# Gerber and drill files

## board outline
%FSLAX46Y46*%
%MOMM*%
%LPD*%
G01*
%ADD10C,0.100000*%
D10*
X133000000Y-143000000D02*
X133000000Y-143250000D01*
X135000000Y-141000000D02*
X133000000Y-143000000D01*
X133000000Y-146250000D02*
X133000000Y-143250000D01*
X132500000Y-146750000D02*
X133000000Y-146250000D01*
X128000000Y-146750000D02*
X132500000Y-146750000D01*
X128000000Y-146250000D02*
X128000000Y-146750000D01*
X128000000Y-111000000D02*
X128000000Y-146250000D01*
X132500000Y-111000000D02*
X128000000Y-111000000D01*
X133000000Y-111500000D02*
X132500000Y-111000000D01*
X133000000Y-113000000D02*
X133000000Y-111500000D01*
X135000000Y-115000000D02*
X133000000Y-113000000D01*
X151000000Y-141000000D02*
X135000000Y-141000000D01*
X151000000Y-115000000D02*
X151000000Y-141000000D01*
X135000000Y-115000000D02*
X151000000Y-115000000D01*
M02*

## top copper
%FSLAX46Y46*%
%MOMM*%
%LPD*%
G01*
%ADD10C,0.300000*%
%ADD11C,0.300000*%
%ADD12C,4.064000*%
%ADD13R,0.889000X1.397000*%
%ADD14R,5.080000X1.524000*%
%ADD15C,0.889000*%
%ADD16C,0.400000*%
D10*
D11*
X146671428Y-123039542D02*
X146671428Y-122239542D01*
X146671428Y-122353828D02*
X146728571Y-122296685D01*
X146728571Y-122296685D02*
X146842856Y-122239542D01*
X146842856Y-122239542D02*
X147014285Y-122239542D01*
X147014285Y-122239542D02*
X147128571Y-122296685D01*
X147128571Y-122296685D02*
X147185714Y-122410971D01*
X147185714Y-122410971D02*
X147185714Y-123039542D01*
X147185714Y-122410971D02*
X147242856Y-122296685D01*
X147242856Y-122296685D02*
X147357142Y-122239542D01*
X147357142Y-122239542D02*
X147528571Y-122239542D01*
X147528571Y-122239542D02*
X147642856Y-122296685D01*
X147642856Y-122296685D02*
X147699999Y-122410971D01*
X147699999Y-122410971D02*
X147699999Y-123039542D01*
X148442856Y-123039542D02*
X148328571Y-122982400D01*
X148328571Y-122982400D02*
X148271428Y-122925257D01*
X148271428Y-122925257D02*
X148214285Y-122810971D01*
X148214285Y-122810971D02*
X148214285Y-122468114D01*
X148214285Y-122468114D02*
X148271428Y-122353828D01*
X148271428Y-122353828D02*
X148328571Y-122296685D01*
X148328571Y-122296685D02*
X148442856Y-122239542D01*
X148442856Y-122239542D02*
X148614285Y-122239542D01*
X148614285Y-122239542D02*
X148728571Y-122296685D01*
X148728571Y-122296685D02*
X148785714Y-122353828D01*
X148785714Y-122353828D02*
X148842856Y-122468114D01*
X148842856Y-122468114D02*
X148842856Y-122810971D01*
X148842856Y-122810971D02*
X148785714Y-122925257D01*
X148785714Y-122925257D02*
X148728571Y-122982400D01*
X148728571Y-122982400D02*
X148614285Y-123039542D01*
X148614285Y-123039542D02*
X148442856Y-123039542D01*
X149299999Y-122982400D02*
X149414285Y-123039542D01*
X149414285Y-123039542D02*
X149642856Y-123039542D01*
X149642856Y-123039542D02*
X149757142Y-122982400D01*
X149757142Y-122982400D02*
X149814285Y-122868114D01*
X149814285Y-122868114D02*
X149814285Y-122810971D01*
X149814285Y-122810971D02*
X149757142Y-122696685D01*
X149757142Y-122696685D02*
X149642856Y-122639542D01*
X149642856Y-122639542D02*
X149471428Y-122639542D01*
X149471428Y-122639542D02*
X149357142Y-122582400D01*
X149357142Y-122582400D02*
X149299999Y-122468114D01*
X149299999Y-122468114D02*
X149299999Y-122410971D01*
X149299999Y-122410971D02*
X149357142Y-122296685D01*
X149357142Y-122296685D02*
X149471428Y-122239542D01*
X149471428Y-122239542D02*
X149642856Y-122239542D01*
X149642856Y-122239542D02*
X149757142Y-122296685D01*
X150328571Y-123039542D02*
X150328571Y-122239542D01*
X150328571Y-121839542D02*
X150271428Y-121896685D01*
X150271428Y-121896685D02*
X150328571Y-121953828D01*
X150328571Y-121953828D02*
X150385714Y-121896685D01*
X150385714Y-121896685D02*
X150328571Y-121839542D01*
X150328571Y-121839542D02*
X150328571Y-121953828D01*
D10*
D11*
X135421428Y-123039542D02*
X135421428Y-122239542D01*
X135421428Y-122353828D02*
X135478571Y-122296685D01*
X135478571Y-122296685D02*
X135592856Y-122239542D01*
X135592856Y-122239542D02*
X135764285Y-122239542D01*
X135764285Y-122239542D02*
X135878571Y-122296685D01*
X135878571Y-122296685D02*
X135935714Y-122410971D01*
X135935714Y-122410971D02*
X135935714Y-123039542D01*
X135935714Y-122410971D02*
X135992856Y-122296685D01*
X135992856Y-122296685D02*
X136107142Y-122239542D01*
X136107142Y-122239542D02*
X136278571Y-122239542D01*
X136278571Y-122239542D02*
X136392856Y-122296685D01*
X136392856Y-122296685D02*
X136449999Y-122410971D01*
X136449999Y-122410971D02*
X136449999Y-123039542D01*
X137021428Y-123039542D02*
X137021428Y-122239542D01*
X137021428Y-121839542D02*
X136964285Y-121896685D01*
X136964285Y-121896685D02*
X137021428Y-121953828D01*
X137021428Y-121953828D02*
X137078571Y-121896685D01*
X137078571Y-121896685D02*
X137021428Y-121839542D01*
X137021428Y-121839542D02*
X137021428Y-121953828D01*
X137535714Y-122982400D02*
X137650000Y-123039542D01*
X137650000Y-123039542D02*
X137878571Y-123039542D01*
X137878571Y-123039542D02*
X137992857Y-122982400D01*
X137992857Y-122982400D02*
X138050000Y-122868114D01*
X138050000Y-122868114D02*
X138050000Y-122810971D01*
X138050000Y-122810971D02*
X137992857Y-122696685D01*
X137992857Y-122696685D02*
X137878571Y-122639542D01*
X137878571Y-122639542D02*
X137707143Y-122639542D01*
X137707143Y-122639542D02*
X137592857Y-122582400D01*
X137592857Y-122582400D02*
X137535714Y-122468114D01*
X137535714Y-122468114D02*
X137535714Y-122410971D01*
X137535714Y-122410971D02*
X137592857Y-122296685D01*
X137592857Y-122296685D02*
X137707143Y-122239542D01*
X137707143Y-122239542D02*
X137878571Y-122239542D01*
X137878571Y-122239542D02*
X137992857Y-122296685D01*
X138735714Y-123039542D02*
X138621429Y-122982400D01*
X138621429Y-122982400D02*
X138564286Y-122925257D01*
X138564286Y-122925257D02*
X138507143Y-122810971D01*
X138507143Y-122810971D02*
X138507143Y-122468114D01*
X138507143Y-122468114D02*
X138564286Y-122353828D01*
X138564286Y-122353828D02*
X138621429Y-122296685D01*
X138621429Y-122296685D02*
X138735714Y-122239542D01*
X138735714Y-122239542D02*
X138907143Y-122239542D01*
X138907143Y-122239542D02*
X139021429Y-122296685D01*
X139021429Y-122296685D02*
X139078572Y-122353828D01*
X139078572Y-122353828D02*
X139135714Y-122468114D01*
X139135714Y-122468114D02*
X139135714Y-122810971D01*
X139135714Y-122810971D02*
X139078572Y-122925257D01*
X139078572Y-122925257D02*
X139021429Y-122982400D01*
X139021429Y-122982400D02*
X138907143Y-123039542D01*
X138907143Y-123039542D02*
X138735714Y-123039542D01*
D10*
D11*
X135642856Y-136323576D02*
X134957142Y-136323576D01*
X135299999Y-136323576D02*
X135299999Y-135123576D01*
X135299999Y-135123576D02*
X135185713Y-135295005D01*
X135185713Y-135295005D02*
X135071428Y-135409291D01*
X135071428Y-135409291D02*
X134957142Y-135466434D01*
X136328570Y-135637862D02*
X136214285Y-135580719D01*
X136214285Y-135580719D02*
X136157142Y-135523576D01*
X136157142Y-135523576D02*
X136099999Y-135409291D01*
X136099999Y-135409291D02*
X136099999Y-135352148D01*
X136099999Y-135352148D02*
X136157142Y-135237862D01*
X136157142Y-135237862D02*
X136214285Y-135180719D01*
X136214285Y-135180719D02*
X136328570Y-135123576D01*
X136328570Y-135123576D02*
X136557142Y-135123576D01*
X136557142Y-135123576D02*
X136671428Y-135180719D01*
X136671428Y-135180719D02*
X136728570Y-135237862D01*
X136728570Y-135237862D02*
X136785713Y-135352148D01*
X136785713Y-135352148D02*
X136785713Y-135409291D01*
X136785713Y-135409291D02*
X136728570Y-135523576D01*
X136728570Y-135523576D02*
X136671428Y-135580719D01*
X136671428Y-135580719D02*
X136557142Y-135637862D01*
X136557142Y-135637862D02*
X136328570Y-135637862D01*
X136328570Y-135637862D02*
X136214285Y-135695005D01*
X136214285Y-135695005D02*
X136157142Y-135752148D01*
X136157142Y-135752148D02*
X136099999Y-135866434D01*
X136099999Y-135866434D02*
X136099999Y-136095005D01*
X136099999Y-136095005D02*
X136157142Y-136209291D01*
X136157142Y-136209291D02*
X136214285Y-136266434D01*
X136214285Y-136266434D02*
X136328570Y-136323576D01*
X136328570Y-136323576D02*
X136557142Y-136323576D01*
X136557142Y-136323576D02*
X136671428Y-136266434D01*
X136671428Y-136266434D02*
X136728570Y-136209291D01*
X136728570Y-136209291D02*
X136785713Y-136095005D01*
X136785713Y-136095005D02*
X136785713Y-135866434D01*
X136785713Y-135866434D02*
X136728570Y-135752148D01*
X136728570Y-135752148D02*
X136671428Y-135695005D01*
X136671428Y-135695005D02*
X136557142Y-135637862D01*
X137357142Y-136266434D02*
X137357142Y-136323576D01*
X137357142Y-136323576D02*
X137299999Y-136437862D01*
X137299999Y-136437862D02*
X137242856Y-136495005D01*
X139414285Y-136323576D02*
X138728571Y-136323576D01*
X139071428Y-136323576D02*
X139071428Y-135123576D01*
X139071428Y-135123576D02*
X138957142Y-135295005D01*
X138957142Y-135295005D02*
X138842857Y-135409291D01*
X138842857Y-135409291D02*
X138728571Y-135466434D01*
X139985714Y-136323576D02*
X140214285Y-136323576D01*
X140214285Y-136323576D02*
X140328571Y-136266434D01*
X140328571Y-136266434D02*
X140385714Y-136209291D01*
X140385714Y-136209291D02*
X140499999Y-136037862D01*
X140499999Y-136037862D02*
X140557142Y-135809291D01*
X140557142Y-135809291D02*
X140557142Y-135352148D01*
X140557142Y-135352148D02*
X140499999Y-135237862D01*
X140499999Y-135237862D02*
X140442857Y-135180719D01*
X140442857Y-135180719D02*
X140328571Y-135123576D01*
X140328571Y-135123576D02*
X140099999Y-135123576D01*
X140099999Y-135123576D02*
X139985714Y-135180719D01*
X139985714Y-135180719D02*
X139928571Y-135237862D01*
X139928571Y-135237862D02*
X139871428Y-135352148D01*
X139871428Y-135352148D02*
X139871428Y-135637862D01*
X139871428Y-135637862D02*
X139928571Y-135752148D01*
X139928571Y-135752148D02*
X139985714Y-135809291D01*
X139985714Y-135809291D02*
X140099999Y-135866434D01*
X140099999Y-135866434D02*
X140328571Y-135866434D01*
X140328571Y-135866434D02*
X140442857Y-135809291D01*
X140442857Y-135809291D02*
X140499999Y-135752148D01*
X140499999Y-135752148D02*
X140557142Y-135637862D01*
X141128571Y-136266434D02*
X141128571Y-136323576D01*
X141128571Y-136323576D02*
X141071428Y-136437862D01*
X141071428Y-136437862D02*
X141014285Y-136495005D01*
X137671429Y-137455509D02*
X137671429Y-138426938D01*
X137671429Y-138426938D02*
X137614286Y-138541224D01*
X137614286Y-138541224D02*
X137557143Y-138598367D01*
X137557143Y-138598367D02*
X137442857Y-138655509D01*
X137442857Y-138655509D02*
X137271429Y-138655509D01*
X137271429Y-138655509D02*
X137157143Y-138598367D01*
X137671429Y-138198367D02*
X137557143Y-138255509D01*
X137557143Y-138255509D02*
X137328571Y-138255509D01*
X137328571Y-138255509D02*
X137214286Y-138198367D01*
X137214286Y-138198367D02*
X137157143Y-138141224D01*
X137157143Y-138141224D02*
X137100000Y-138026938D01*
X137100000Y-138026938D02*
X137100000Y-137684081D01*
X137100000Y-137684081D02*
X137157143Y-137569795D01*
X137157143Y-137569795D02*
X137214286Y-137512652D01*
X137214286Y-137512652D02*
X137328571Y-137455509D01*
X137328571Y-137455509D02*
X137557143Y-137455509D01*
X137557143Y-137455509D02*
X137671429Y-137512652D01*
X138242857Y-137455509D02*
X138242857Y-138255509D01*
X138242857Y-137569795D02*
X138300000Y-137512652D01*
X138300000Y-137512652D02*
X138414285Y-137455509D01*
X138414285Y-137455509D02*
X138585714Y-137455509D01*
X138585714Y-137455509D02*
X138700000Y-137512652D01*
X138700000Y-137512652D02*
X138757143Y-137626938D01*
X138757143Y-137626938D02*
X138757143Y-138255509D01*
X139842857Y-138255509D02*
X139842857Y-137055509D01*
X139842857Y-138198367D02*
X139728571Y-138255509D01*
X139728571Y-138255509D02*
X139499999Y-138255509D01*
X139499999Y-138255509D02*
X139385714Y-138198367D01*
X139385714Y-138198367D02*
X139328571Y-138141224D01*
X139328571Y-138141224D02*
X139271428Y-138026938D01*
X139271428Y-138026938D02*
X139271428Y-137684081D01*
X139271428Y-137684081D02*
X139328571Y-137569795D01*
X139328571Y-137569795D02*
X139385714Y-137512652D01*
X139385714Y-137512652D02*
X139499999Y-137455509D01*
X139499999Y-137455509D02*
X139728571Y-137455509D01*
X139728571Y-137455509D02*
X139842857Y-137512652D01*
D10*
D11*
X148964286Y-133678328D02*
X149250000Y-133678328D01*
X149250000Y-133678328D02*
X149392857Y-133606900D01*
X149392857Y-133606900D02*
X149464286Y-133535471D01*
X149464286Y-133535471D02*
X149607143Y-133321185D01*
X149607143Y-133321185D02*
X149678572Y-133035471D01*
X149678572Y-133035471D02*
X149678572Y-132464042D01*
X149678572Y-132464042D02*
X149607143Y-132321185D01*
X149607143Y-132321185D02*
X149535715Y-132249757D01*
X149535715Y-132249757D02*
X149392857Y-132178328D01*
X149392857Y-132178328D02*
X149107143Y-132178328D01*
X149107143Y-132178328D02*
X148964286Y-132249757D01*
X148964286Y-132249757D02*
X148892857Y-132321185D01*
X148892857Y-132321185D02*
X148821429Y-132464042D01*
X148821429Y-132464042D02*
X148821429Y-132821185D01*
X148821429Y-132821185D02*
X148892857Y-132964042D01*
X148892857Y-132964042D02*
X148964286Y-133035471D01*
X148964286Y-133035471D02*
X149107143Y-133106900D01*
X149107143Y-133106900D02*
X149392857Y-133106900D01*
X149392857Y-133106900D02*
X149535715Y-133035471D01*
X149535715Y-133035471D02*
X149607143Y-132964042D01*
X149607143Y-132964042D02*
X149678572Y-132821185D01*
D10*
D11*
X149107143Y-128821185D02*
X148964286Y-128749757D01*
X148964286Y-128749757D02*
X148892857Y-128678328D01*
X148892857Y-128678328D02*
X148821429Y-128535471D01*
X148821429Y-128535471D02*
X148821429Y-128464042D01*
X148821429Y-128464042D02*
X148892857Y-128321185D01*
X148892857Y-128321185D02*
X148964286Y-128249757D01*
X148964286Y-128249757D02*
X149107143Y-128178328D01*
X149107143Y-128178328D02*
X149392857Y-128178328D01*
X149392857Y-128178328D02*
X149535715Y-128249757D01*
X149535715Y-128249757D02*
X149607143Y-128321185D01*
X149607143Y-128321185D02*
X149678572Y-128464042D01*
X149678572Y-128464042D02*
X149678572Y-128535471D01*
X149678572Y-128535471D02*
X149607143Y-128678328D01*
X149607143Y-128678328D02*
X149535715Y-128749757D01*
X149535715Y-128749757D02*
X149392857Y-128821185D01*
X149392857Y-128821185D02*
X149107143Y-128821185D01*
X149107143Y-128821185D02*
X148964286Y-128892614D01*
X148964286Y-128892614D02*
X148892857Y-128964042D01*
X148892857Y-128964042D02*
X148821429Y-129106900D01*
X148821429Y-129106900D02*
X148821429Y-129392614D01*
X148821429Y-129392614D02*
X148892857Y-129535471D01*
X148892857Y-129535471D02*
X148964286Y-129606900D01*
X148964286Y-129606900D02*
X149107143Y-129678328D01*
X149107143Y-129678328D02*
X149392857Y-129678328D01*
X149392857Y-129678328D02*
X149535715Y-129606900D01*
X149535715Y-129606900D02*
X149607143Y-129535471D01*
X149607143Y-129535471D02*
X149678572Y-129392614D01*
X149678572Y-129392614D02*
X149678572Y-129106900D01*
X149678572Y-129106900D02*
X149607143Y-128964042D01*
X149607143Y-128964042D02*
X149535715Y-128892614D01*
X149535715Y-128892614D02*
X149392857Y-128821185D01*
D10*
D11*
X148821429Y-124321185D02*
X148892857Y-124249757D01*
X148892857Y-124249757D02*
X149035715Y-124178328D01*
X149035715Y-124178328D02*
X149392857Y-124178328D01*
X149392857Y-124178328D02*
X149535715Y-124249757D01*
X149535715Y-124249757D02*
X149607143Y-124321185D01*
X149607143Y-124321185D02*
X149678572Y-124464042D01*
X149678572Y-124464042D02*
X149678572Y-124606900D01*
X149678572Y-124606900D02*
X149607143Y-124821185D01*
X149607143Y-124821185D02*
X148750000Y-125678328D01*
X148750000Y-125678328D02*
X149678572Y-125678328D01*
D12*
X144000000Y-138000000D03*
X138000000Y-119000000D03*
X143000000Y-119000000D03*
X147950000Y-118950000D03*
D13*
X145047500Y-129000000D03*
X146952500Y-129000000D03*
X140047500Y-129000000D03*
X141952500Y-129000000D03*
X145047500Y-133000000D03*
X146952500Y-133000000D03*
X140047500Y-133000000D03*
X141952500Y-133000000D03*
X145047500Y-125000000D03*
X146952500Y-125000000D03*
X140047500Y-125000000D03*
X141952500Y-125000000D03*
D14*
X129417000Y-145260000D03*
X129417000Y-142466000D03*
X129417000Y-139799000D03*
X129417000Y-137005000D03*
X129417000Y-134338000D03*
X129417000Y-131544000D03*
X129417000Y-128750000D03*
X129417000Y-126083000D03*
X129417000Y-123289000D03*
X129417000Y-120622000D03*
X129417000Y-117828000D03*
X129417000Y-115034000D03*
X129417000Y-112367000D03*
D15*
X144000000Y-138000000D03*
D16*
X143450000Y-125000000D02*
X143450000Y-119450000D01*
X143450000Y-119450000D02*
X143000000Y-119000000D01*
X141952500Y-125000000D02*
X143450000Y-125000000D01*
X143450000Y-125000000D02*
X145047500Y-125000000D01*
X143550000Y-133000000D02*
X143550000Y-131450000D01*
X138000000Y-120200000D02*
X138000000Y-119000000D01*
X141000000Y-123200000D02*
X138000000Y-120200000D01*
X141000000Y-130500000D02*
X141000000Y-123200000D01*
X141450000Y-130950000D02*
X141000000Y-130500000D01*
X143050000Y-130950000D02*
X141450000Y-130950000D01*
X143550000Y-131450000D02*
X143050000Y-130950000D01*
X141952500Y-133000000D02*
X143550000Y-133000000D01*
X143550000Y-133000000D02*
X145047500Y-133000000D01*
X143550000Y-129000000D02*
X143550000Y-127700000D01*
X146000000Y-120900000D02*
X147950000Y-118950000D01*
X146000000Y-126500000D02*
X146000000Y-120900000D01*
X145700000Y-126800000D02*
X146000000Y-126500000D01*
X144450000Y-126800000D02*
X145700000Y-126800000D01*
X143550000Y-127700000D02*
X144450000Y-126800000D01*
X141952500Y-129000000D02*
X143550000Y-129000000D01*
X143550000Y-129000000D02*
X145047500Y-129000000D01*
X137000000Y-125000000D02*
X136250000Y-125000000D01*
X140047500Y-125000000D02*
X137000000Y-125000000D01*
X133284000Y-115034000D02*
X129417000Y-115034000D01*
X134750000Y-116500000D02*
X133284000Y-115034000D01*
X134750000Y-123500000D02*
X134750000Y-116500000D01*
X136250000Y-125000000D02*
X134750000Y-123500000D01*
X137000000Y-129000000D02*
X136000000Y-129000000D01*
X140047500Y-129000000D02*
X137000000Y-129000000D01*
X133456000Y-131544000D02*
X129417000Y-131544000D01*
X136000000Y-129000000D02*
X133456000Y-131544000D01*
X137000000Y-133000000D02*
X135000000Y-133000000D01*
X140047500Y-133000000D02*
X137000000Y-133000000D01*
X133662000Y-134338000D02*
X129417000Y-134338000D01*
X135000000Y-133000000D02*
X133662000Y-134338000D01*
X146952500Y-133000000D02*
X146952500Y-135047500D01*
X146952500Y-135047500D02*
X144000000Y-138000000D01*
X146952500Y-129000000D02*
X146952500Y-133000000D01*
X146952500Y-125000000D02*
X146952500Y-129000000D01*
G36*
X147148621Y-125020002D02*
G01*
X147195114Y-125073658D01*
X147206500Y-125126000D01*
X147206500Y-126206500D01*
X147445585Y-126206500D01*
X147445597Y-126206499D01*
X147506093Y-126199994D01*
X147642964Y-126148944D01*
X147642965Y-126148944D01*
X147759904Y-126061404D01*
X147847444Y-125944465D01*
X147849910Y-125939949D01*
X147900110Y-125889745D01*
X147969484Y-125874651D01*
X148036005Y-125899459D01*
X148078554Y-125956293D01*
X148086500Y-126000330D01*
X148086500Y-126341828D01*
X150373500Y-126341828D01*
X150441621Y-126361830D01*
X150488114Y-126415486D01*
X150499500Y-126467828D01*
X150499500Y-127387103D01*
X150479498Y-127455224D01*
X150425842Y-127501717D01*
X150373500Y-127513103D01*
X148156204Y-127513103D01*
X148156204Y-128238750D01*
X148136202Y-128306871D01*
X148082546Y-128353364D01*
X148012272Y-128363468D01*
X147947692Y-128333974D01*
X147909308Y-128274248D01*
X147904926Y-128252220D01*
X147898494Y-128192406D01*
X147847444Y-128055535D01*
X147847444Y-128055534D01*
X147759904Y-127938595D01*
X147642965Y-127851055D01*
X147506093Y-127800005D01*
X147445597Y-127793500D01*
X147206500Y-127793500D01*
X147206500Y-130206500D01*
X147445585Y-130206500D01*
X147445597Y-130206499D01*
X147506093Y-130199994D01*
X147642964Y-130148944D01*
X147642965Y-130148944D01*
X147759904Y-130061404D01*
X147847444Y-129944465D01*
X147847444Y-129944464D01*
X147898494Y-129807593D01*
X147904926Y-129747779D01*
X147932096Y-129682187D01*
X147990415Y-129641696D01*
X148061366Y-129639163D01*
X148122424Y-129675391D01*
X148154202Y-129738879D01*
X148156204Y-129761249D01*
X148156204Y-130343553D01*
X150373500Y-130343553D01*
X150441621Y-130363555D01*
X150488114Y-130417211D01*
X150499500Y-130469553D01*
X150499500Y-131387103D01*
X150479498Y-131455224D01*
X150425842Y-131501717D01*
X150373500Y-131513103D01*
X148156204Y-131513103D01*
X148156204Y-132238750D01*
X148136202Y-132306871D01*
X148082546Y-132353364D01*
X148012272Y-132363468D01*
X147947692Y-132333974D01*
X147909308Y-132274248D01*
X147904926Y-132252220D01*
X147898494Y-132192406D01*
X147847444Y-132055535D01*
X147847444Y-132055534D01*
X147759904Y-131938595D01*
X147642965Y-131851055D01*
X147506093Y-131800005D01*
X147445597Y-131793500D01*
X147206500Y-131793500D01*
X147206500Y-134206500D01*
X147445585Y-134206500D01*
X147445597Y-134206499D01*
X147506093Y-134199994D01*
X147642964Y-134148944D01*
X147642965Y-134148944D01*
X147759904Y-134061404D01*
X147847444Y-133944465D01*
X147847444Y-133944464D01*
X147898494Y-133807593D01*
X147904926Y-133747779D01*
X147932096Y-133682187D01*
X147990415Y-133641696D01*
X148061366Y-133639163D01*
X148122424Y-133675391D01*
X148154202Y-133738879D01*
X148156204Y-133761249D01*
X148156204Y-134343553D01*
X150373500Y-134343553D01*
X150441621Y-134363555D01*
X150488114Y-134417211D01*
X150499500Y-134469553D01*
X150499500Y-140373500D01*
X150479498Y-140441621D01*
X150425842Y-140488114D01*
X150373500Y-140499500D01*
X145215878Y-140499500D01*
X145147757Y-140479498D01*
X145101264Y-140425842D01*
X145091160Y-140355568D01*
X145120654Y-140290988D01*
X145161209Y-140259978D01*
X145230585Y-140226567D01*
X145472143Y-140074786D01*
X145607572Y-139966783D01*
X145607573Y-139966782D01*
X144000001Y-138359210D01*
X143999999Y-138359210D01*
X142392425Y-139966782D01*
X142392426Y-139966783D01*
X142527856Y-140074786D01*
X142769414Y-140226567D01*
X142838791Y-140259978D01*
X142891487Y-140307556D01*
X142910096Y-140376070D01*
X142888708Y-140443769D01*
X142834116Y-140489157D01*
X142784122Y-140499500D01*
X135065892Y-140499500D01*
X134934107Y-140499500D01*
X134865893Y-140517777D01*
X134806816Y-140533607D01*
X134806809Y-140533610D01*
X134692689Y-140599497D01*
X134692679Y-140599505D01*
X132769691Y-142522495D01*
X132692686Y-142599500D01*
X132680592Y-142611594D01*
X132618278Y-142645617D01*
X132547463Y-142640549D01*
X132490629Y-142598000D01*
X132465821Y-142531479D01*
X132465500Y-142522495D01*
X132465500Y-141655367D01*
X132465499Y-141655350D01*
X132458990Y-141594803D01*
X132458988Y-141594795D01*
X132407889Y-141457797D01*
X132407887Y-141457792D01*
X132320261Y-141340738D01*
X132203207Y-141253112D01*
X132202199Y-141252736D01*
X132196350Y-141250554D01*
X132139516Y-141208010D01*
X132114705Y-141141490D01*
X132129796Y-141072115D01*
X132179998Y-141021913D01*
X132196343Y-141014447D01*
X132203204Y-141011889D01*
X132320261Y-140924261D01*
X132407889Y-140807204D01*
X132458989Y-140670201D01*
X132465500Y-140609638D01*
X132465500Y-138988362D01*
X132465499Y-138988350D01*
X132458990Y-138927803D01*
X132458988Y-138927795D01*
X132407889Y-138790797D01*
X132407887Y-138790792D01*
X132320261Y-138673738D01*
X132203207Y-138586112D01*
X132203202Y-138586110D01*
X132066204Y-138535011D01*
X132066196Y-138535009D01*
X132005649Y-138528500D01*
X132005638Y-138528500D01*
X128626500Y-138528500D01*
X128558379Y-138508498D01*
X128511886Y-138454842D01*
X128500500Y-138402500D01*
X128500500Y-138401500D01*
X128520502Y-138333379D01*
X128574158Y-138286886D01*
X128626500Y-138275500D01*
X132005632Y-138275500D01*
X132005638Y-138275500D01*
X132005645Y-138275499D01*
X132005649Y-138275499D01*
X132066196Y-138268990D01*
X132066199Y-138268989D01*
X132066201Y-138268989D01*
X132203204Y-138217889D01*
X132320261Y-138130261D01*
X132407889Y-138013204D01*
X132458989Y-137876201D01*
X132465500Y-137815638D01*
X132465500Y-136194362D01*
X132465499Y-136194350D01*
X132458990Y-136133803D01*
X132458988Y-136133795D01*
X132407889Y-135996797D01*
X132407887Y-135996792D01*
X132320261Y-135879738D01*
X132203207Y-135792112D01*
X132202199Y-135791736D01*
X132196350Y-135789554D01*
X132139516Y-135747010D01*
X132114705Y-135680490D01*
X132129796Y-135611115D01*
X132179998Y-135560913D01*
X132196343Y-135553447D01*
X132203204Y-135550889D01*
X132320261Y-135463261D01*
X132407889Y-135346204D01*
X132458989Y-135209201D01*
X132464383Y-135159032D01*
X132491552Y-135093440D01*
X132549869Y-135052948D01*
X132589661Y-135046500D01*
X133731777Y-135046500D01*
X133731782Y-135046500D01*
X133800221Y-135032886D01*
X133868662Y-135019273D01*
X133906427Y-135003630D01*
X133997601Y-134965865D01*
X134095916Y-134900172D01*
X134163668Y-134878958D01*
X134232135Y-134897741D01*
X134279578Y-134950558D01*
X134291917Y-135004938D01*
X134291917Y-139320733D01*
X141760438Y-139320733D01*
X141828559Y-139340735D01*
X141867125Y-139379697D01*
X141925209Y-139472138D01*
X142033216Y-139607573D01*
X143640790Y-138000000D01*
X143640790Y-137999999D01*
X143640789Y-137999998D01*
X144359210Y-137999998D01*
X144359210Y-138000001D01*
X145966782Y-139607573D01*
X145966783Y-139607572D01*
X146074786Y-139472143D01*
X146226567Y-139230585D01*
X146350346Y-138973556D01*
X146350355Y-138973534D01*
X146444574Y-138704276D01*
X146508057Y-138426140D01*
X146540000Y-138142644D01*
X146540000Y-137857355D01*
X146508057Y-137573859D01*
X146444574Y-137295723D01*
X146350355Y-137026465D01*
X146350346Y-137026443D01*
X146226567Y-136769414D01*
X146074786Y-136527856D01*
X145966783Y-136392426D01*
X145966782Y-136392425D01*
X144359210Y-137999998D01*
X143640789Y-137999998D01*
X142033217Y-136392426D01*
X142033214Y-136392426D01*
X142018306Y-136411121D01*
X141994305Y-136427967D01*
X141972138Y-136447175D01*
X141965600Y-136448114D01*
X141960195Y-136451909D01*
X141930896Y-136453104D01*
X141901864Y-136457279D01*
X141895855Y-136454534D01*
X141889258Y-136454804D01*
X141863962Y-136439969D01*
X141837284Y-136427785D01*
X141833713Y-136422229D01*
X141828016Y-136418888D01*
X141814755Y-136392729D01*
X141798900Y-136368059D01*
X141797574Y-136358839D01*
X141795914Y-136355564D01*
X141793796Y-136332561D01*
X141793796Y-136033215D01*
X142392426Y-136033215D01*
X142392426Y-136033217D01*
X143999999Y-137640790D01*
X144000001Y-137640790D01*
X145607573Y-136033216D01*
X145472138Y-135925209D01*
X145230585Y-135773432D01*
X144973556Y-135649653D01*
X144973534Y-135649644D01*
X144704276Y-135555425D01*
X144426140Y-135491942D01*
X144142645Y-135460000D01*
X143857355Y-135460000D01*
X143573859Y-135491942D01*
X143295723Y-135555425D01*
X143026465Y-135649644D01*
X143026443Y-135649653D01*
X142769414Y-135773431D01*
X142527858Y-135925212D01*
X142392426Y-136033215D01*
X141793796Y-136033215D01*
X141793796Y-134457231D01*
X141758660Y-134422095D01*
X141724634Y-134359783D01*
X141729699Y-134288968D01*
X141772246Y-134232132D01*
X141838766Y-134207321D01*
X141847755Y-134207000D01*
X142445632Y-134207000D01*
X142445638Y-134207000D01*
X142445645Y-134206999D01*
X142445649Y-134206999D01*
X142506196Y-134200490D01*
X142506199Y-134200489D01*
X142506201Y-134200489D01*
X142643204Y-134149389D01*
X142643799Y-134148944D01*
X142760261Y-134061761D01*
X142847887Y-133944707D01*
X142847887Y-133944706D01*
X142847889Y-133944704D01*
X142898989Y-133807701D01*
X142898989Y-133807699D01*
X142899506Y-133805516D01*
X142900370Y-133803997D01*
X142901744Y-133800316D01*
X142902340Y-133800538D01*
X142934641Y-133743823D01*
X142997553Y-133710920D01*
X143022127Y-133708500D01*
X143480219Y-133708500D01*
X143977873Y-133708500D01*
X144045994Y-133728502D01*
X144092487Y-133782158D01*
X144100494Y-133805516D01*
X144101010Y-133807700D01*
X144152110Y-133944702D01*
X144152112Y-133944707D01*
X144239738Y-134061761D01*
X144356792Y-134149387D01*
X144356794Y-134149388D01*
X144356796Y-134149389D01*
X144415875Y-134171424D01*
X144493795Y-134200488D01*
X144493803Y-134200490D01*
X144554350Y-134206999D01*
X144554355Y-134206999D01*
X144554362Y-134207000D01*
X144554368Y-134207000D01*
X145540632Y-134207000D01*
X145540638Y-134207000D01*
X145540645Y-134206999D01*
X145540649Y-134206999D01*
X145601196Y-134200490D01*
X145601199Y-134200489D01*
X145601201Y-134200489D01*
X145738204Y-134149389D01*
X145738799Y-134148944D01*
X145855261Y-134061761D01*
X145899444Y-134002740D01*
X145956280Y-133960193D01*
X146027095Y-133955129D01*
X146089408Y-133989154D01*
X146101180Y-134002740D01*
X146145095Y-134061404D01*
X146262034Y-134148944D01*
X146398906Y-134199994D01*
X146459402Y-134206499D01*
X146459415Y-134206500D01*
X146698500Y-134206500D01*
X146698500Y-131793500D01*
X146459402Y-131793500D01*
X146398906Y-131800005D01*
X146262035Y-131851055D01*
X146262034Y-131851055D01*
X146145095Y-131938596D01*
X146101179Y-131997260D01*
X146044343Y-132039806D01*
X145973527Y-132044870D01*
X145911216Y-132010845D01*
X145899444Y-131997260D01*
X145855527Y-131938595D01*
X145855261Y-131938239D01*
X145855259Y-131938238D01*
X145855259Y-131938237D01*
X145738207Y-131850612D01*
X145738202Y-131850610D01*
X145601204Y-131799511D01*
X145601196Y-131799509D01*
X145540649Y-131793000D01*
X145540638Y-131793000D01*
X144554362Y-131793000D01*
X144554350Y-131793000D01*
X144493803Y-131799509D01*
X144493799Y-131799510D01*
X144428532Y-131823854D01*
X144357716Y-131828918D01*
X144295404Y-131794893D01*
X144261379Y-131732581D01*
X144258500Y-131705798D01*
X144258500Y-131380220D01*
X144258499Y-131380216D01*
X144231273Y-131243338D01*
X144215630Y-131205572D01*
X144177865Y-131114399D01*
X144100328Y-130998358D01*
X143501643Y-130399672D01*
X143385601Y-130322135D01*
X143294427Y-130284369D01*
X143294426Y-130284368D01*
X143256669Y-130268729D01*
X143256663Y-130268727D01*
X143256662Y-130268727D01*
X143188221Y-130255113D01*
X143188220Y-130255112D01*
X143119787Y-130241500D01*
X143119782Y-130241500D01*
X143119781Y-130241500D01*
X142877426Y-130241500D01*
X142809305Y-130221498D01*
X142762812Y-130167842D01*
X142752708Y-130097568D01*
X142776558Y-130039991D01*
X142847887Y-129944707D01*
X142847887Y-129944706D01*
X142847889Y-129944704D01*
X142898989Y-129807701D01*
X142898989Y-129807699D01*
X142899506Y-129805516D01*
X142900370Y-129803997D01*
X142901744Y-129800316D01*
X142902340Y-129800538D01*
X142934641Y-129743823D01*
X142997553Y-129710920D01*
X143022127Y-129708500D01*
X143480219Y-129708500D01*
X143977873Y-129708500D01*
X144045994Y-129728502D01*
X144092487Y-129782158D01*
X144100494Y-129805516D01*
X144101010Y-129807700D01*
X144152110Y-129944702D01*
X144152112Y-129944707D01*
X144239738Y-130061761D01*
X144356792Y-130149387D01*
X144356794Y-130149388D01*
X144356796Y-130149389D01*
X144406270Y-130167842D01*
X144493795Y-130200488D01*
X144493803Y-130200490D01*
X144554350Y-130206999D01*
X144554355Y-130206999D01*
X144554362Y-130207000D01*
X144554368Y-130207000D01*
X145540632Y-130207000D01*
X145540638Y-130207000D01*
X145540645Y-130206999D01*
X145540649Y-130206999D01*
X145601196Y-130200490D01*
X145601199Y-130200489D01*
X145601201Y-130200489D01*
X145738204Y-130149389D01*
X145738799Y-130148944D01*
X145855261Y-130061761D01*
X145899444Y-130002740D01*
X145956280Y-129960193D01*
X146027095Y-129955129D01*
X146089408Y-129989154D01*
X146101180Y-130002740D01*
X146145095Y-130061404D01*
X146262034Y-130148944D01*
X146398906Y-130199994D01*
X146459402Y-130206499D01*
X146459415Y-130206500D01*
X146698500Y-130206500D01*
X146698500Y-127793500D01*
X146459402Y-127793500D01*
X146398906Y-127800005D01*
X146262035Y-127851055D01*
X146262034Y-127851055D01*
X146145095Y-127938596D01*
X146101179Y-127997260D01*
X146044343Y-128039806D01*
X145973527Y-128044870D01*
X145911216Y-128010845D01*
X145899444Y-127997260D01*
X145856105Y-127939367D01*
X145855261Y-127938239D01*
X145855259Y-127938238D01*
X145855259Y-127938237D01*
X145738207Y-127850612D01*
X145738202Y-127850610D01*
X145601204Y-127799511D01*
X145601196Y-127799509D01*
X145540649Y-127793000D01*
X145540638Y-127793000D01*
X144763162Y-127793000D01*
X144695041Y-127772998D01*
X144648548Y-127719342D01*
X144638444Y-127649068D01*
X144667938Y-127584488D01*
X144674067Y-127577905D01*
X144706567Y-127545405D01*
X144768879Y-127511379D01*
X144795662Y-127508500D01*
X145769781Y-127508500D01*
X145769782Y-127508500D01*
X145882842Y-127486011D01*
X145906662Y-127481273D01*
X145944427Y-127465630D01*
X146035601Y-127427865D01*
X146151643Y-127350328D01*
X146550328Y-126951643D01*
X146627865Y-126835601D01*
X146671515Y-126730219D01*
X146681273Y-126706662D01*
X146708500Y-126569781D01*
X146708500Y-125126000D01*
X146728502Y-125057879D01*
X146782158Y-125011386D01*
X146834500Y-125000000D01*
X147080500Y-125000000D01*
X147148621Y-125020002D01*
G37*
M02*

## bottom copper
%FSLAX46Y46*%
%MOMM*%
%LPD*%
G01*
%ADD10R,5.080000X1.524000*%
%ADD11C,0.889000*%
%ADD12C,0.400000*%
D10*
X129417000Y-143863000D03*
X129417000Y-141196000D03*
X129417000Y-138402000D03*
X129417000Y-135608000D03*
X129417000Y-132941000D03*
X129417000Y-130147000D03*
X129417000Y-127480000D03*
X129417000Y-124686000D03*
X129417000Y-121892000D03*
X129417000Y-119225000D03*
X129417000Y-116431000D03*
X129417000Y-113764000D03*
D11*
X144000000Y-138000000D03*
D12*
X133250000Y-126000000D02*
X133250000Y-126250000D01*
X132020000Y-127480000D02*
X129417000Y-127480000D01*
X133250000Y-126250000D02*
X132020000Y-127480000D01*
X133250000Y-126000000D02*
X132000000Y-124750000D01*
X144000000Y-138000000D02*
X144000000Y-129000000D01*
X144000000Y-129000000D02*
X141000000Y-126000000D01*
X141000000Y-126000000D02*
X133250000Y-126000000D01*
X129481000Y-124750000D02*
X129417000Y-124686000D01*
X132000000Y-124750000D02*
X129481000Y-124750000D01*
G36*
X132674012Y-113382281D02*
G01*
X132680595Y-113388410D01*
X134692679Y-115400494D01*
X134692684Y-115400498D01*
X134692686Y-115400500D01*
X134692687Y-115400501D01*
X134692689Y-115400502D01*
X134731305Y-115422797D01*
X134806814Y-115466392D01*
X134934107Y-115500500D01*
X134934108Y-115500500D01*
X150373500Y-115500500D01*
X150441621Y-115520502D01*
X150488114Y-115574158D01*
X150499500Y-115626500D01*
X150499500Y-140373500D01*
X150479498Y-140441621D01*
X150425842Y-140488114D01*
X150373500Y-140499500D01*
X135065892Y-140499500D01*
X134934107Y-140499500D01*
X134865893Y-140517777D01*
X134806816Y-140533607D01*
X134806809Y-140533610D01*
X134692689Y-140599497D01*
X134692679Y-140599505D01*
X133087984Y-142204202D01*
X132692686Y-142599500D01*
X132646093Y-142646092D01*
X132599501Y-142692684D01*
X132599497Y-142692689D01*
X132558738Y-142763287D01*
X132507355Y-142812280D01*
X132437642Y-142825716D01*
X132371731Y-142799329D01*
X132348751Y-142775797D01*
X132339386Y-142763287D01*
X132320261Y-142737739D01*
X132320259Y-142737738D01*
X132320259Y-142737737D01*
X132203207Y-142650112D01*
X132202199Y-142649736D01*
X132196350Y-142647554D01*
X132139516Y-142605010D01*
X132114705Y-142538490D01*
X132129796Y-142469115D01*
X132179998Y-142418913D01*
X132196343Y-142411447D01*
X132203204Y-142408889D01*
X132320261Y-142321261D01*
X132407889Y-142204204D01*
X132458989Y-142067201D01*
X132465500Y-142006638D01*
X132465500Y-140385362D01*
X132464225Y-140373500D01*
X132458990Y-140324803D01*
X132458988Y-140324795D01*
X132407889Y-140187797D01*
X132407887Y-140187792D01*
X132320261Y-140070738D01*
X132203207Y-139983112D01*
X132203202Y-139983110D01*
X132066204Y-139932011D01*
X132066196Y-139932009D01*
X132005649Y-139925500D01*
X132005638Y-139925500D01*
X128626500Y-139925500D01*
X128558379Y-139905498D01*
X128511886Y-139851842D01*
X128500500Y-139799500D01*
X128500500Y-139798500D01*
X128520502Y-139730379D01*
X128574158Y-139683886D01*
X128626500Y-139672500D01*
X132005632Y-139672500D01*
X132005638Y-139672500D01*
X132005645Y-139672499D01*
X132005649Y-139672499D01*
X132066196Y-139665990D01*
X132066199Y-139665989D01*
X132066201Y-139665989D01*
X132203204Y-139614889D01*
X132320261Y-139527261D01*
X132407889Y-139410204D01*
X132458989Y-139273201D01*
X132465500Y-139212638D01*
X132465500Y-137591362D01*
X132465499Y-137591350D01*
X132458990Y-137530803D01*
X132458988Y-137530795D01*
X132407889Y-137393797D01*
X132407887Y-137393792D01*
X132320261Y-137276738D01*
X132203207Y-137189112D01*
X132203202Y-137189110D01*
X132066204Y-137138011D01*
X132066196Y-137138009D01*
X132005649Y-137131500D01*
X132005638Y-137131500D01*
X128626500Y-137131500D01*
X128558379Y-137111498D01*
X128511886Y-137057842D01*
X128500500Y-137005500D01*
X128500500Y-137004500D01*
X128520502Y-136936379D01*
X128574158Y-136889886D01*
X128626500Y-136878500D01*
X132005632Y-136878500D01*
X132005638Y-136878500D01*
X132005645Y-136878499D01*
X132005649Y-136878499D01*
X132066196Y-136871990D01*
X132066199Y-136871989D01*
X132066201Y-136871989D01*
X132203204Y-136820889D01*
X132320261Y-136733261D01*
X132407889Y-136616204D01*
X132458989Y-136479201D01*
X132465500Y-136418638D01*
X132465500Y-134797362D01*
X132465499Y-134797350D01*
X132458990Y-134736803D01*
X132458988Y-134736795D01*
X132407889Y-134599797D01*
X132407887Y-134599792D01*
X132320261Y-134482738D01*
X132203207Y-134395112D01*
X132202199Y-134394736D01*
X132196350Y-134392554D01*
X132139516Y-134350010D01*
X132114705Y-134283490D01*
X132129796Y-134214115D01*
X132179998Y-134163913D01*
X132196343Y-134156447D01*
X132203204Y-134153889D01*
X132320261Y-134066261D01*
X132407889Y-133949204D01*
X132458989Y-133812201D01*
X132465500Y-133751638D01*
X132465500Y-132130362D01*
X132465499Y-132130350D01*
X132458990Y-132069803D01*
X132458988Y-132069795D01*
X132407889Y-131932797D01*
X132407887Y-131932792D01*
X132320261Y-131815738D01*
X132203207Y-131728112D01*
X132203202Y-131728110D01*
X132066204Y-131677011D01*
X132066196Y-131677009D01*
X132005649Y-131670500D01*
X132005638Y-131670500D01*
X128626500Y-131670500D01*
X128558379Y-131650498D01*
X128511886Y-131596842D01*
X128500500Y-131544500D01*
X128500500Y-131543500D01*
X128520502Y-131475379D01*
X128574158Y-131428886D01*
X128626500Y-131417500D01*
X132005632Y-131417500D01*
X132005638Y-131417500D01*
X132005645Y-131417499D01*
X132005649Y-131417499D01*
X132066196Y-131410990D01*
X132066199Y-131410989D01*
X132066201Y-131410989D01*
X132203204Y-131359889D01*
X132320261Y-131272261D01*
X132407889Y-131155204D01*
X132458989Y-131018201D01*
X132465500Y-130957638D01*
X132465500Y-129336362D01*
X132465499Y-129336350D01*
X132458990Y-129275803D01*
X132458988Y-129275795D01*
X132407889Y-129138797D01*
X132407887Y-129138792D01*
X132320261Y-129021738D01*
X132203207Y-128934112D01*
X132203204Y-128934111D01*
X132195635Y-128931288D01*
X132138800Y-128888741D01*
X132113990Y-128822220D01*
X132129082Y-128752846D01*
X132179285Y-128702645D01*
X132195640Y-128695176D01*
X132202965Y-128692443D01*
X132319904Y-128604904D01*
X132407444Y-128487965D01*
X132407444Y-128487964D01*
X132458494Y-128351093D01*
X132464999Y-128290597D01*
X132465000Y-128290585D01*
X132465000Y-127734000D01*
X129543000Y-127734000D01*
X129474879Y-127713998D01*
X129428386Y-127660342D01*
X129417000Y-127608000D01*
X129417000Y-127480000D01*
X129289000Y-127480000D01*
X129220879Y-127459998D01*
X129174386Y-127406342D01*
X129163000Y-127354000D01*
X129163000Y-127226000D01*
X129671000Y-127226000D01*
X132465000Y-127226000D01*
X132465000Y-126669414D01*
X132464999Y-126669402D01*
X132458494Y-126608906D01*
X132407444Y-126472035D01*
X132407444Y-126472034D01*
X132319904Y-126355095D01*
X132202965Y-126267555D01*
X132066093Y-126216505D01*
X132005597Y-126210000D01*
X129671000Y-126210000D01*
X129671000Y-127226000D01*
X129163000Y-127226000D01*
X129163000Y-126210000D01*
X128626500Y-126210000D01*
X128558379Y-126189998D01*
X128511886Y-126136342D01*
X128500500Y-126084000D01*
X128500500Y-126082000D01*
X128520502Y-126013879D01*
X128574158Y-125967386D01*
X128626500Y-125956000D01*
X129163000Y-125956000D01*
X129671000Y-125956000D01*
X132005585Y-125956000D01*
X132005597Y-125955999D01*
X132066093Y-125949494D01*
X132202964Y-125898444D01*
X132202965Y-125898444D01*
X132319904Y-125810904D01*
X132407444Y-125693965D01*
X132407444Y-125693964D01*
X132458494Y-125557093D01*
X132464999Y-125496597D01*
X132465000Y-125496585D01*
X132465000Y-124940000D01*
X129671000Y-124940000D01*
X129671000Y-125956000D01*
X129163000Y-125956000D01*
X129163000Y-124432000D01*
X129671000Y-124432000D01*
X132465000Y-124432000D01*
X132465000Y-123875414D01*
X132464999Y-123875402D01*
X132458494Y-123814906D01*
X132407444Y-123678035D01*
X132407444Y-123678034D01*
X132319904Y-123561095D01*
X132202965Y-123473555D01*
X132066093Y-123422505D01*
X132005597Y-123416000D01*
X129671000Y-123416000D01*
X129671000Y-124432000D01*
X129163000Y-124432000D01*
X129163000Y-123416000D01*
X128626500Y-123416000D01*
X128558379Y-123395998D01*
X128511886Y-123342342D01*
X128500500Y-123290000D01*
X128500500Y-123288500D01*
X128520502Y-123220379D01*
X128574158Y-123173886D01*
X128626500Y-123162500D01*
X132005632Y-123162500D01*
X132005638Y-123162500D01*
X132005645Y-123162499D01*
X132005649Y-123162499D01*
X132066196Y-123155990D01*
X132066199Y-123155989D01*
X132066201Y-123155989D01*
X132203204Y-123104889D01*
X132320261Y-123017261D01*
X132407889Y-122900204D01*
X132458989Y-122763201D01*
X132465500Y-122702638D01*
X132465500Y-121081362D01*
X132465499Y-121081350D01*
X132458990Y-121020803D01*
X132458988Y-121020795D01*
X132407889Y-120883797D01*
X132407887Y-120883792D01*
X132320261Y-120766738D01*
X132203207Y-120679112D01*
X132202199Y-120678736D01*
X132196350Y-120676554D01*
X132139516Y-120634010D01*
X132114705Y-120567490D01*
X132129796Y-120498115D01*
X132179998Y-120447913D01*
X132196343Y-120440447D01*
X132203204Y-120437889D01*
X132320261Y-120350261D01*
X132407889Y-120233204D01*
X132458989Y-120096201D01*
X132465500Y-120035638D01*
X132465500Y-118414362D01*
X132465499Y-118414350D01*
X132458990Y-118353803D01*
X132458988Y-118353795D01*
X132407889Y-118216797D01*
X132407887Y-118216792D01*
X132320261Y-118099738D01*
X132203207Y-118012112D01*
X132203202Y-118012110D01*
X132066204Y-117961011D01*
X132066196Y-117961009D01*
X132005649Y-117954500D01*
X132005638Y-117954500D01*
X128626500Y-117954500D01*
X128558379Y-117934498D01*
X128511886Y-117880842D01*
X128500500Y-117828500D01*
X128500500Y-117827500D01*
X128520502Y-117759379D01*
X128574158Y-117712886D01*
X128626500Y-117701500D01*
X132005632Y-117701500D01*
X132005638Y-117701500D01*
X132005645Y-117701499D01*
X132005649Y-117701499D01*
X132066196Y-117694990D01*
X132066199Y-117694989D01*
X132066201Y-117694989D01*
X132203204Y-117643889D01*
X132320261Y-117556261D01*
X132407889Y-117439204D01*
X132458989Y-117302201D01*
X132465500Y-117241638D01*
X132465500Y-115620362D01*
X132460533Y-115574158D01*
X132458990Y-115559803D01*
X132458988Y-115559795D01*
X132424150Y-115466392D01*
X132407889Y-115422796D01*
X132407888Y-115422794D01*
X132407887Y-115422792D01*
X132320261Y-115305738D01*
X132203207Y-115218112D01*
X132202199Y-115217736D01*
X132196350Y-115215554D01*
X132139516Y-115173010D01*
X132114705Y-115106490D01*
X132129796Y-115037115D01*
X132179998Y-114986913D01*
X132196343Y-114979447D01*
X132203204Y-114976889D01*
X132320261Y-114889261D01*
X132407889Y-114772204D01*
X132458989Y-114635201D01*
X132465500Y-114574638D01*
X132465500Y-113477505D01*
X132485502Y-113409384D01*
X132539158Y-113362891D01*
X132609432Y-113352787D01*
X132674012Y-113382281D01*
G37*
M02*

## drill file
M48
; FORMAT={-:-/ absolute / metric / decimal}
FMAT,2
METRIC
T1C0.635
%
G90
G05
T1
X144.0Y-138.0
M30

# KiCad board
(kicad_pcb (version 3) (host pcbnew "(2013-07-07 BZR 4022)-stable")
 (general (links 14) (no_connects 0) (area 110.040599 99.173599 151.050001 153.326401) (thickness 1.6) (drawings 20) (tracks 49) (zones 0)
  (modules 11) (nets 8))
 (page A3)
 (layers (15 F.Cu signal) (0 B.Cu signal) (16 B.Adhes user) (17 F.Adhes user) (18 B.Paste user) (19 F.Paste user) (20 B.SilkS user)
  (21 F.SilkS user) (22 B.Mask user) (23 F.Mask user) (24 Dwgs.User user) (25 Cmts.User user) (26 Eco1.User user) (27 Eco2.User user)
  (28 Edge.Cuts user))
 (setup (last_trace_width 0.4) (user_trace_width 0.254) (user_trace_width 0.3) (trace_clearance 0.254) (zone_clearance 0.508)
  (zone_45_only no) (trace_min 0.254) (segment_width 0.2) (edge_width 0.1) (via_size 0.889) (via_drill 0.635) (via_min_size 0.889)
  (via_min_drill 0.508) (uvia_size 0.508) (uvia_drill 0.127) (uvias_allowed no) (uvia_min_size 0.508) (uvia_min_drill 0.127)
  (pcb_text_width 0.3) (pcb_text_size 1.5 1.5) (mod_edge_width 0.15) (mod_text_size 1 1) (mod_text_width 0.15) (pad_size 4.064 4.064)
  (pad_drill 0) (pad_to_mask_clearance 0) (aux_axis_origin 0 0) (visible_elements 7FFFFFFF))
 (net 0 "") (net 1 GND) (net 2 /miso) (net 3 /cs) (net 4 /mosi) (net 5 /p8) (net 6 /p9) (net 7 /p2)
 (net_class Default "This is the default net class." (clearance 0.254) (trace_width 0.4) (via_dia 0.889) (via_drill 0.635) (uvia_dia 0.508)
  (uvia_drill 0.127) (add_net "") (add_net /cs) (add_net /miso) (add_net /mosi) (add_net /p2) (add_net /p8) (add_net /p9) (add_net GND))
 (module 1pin (layer F.Cu) (at 144 138)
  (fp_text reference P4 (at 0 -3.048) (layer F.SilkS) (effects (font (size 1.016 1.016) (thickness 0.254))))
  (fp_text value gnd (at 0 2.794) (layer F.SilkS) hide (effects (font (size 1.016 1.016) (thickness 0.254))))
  (pad 1 smd circle (at 0 0) (size 4.064 4.064) (layers F.Cu F.Paste F.Mask) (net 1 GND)))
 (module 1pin (layer F.Cu) (at 138 119)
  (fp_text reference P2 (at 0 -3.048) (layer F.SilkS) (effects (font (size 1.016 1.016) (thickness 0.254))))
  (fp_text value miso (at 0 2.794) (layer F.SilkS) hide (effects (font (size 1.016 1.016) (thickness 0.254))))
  (pad 1 smd circle (at 0 0) (size 4.064 4.064) (layers F.Cu F.Paste F.Mask) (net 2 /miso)))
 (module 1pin (layer F.Cu) (at 143 119)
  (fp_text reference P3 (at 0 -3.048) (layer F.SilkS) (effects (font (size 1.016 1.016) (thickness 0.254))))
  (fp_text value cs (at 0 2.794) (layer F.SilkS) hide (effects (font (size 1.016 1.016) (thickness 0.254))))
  (pad 1 smd circle (at 0 0) (size 4.064 4.064) (layers F.Cu F.Paste F.Mask) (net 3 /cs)))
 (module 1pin (layer F.Cu) (at 147.95 118.95)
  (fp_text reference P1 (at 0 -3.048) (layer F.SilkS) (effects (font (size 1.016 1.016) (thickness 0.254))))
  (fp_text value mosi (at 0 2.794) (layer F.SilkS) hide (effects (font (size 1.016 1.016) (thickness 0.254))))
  (pad 1 smd circle (at 0 0) (size 4.064 4.064) (layers F.Cu F.Paste F.Mask) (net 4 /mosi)))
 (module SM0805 (layer F.Cu) (at 146 129)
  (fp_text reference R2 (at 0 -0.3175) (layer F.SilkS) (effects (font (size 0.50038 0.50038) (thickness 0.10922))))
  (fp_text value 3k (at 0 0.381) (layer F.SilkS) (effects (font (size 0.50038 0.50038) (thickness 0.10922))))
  (pad 1 smd rect (at -0.9525 0) (size 0.889 1.397) (layers F.Cu F.Paste F.Mask) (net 4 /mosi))
  (pad 2 smd rect (at 0.9525 0) (size 0.889 1.397) (layers F.Cu F.Paste F.Mask) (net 1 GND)))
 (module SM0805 (layer F.Cu) (at 141 129)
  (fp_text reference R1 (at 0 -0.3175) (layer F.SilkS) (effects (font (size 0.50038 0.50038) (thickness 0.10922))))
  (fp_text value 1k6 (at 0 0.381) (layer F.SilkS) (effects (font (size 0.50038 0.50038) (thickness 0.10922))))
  (pad 1 smd rect (at -0.9525 0) (size 0.889 1.397) (layers F.Cu F.Paste F.Mask) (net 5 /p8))
  (pad 2 smd rect (at 0.9525 0) (size 0.889 1.397) (layers F.Cu F.Paste F.Mask) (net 4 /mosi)))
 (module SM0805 (layer F.Cu) (at 146 133)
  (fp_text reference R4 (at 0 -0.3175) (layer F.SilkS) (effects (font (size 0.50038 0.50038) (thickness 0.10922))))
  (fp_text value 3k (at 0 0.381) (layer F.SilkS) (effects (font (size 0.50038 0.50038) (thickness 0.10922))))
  (pad 1 smd rect (at -0.9525 0) (size 0.889 1.397) (layers F.Cu F.Paste F.Mask) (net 2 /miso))
  (pad 2 smd rect (at 0.9525 0) (size 0.889 1.397) (layers F.Cu F.Paste F.Mask) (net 1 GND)))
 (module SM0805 (layer F.Cu) (at 141 133)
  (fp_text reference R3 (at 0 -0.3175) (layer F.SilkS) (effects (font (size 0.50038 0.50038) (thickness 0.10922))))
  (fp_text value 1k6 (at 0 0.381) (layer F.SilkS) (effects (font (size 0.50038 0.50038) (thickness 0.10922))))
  (pad 1 smd rect (at -0.9525 0) (size 0.889 1.397) (layers F.Cu F.Paste F.Mask) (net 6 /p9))
  (pad 2 smd rect (at 0.9525 0) (size 0.889 1.397) (layers F.Cu F.Paste F.Mask) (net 2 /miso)))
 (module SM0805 (layer F.Cu) (at 146 125)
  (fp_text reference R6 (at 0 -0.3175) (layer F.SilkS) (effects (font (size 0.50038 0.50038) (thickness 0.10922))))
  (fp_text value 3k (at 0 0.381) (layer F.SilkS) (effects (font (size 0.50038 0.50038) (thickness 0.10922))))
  (pad 1 smd rect (at -0.9525 0) (size 0.889 1.397) (layers F.Cu F.Paste F.Mask) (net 3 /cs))
  (pad 2 smd rect (at 0.9525 0) (size 0.889 1.397) (layers F.Cu F.Paste F.Mask) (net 1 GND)))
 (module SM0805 (layer F.Cu) (at 141 125)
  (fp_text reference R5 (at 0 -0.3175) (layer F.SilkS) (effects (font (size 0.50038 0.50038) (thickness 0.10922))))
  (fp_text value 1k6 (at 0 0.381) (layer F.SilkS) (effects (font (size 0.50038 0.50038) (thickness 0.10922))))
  (pad 1 smd rect (at -0.9525 0) (size 0.889 1.397) (layers F.Cu F.Paste F.Mask) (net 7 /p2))
  (pad 2 smd rect (at 0.9525 0) (size 0.889 1.397) (layers F.Cu F.Paste F.Mask) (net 3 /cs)))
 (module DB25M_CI (layer F.Cu) (at 126.75 128.75 90)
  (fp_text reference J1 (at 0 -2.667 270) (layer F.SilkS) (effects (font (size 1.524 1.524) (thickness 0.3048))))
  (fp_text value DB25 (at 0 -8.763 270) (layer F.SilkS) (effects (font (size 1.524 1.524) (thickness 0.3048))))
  (pad 13 connect rect (at -16.51 2.667 180) (size 5.08 1.524) (layers F.Cu F.Mask))
  (pad 12 connect rect (at -13.716 2.667 180) (size 5.08 1.524) (layers F.Cu F.Mask))
  (pad 11 connect rect (at -11.049 2.667 180) (size 5.08 1.524) (layers F.Cu F.Mask))
  (pad 10 connect rect (at -8.255 2.667 180) (size 5.08 1.524) (layers F.Cu F.Mask))
  (pad 9 connect rect (at -5.588 2.667 180) (size 5.08 1.524) (layers F.Cu F.Mask) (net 6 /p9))
  (pad 8 connect rect (at -2.794 2.667 180) (size 5.08 1.524) (layers F.Cu F.Mask) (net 5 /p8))
  (pad 7 connect rect (at 0 2.667 180) (size 5.08 1.524) (layers F.Cu F.Mask))
  (pad 6 connect rect (at 2.667 2.667 180) (size 5.08 1.524) (layers F.Cu F.Mask))
  (pad 5 connect rect (at 5.461 2.667 180) (size 5.08 1.524) (layers F.Cu F.Mask))
  (pad 4 connect rect (at 8.128 2.667 180) (size 5.08 1.524) (layers F.Cu F.Mask))
  (pad 3 connect rect (at 10.922 2.667 180) (size 5.08 1.524) (layers F.Cu F.Mask))
  (pad 2 connect rect (at 13.716 2.667 180) (size 5.08 1.524) (layers F.Cu F.Mask) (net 7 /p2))
  (pad 1 connect rect (at 16.383 2.667 180) (size 5.08 1.524) (layers F.Cu F.Mask))
  (pad 25 connect rect (at -15.113 2.667 180) (size 5.08 1.524) (layers B.Cu B.Mask))
  (pad 24 connect rect (at -12.446 2.667 180) (size 5.08 1.524) (layers B.Cu B.Mask))
  (pad 23 connect rect (at -9.652 2.667 180) (size 5.08 1.524) (layers B.Cu B.Mask))
  (pad 22 connect rect (at -6.858 2.667 180) (size 5.08 1.524) (layers B.Cu B.Mask))
  (pad 21 connect rect (at -4.191 2.667 180) (size 5.08 1.524) (layers B.Cu B.Mask))
  (pad 20 connect rect (at -1.397 2.667 180) (size 5.08 1.524) (layers B.Cu B.Mask))
  (pad 19 connect rect (at 1.27 2.667 180) (size 5.08 1.524) (layers B.Cu B.Mask) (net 1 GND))
  (pad 18 connect rect (at 4.064 2.667 180) (size 5.08 1.524) (layers B.Cu B.Mask) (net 1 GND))
  (pad 17 connect rect (at 6.858 2.667 180) (size 5.08 1.524) (layers B.Cu B.Mask))
  (pad 16 connect rect (at 9.525 2.667 180) (size 5.08 1.524) (layers B.Cu B.Mask))
  (pad 15 connect rect (at 12.319 2.667 180) (size 5.08 1.524) (layers B.Cu B.Mask))
  (pad 14 connect rect (at 14.986 2.667 180) (size 5.08 1.524) (layers B.Cu B.Mask)))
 (gr_line (start 133 143) (end 133 143.25) (angle 90) (layer Edge.Cuts) (width 0.1))
 (gr_line (start 135 141) (end 133 143) (angle 90) (layer Edge.Cuts) (width 0.1))
 (gr_line (start 133 146.25) (end 133 143.25) (angle 90) (layer Edge.Cuts) (width 0.1))
 (gr_line (start 132.5 146.75) (end 133 146.25) (angle 90) (layer Edge.Cuts) (width 0.1))
 (gr_line (start 128 146.75) (end 132.5 146.75) (angle 90) (layer Edge.Cuts) (width 0.1))
 (gr_line (start 128 146.25) (end 128 146.75) (angle 90) (layer Edge.Cuts) (width 0.1))
 (gr_line (start 128 111) (end 128 146.25) (angle 90) (layer Edge.Cuts) (width 0.1))
 (gr_line (start 132.5 111) (end 128 111) (angle 90) (layer Edge.Cuts) (width 0.1))
 (gr_line (start 133 111.5) (end 132.5 111) (angle 90) (layer Edge.Cuts) (width 0.1))
 (gr_line (start 133 113) (end 133 111.5) (angle 90) (layer Edge.Cuts) (width 0.1))
 (gr_line (start 135 115) (end 133 113) (angle 90) (layer Edge.Cuts) (width 0.1))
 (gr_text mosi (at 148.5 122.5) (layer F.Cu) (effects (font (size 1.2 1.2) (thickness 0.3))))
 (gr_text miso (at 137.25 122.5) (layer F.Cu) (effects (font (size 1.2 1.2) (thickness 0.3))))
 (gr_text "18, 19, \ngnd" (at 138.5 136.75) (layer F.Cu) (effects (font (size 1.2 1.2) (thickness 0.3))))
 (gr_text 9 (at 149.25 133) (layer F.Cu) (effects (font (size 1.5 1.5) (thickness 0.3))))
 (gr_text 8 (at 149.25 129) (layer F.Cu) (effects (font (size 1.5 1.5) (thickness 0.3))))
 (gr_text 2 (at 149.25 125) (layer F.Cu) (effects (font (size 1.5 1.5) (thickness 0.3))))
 (gr_line (start 151 141) (end 135 141) (angle 90) (layer Edge.Cuts) (width 0.1))
 (gr_line (start 151 115) (end 151 141) (angle 90) (layer Edge.Cuts) (width 0.1))
 (gr_line (start 135 115) (end 151 115) (angle 90) (layer Edge.Cuts) (width 0.1))
 (segment (start 143.45 125) (end 143.45 119.45) (width 0.4) (layer F.Cu) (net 3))
 (segment (start 143.45 119.45) (end 143 119) (width 0.4) (layer F.Cu) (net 3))
 (segment (start 141.9525 125) (end 143.45 125) (width 0.4) (layer F.Cu) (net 3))
 (segment (start 143.45 125) (end 145.0475 125) (width 0.4) (layer F.Cu) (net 3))
 (segment (start 143.55 133) (end 143.55 131.45) (width 0.4) (layer F.Cu) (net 2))
 (segment (start 138 120.2) (end 138 119) (width 0.4) (layer F.Cu) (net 2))
 (segment (start 141 123.2) (end 138 120.2) (width 0.4) (layer F.Cu) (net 2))
 (segment (start 141 130.5) (end 141 123.2) (width 0.4) (layer F.Cu) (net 2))
 (segment (start 141.45 130.95) (end 141 130.5) (width 0.4) (layer F.Cu) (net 2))
 (segment (start 143.05 130.95) (end 141.45 130.95) (width 0.4) (layer F.Cu) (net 2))
 (segment (start 143.55 131.45) (end 143.05 130.95) (width 0.4) (layer F.Cu) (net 2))
 (segment (start 141.9525 133) (end 143.55 133) (width 0.4) (layer F.Cu) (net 2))
 (segment (start 143.55 133) (end 145.0475 133) (width 0.4) (layer F.Cu) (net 2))
 (segment (start 143.55 129) (end 143.55 127.7) (width 0.4) (layer F.Cu) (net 4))
 (segment (start 146 120.9) (end 147.95 118.95) (width 0.4) (layer F.Cu) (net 4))
 (segment (start 146 126.5) (end 146 120.9) (width 0.4) (layer F.Cu) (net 4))
 (segment (start 145.7 126.8) (end 146 126.5) (width 0.4) (layer F.Cu) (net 4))
 (segment (start 144.45 126.8) (end 145.7 126.8) (width 0.4) (layer F.Cu) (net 4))
 (segment (start 143.55 127.7) (end 144.45 126.8) (width 0.4) (layer F.Cu) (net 4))
 (segment (start 141.9525 129) (end 143.55 129) (width 0.4) (layer F.Cu) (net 4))
 (segment (start 143.55 129) (end 145.0475 129) (width 0.4) (layer F.Cu) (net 4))
 (segment (start 137 125) (end 136.25 125) (width 0.4) (layer F.Cu) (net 7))
 (segment (start 140.0475 125) (end 137 125) (width 0.4) (layer F.Cu) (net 7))
 (segment (start 133.284 115.034) (end 129.417 115.034) (width 0.4) (layer F.Cu) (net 7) (status 800000))
 (segment (start 134.75 116.5) (end 133.284 115.034) (width 0.4) (layer F.Cu) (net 7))
 (segment (start 134.75 123.5) (end 134.75 116.5) (width 0.4) (layer F.Cu) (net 7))
 (segment (start 136.25 125) (end 134.75 123.5) (width 0.4) (layer F.Cu) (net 7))
 (segment (start 137 129) (end 136 129) (width 0.4) (layer F.Cu) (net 5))
 (segment (start 140.0475 129) (end 137 129) (width 0.4) (layer F.Cu) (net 5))
 (segment (start 133.456 131.544) (end 129.417 131.544) (width 0.4) (layer F.Cu) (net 5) (status 800000))
 (segment (start 136 129) (end 133.456 131.544) (width 0.4) (layer F.Cu) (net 5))
 (segment (start 137 133) (end 135 133) (width 0.4) (layer F.Cu) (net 6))
 (segment (start 140.0475 133) (end 137 133) (width 0.4) (layer F.Cu) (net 6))
 (segment (start 133.662 134.338) (end 129.417 134.338) (width 0.4) (layer F.Cu) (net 6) (status 800000))
 (segment (start 135 133) (end 133.662 134.338) (width 0.4) (layer F.Cu) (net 6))
 (segment (start 133.25 126) (end 133.25 126.25) (width 0.4) (layer B.Cu) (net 1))
 (segment (start 132.02 127.48) (end 129.417 127.48) (width 0.4) (layer B.Cu) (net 1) (status 800000))
 (segment (start 133.25 126.25) (end 132.02 127.48) (width 0.4) (layer B.Cu) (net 1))
 (segment (start 133.25 126) (end 132 124.75) (width 0.4) (layer B.Cu) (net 1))
 (segment (start 144 138) (end 144 129) (width 0.4) (layer B.Cu) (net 1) (status 400000))
 (segment (start 144 129) (end 141 126) (width 0.4) (layer B.Cu) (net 1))
 (segment (start 141 126) (end 133.25 126) (width 0.4) (layer B.Cu) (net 1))
 (segment (start 146.9525 133) (end 146.9525 135.0475) (width 0.4) (layer F.Cu) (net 1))
 (segment (start 146.9525 135.0475) (end 144 138) (width 0.4) (layer F.Cu) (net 1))
 (via (at 144 138) (size 0.889) (layers F.Cu B.Cu) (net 1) (status C00000))
 (segment (start 129.481 124.75) (end 129.417 124.686) (width 0.4) (layer B.Cu) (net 1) (status C00000))
 (segment (start 132 124.75) (end 129.481 124.75) (width 0.4) (layer B.Cu) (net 1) (status 800000))
 (segment (start 146.9525 129) (end 146.9525 133) (width 0.4) (layer F.Cu) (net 1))
 (segment (start 146.9525 125) (end 146.9525 129) (width 0.4) (layer F.Cu) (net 1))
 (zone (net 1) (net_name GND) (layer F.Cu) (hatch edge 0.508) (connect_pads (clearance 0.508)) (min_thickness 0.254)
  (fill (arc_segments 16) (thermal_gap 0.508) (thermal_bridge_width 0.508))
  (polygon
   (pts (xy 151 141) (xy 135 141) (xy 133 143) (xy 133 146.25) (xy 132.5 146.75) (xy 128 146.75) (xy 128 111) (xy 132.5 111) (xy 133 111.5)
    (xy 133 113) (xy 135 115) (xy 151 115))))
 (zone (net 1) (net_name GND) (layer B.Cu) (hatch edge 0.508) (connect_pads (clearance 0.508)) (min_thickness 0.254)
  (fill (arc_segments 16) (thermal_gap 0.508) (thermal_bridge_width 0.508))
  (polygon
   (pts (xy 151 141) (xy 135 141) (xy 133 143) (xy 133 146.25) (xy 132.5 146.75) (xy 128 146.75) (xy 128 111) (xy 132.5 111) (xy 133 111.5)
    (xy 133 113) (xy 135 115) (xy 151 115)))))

